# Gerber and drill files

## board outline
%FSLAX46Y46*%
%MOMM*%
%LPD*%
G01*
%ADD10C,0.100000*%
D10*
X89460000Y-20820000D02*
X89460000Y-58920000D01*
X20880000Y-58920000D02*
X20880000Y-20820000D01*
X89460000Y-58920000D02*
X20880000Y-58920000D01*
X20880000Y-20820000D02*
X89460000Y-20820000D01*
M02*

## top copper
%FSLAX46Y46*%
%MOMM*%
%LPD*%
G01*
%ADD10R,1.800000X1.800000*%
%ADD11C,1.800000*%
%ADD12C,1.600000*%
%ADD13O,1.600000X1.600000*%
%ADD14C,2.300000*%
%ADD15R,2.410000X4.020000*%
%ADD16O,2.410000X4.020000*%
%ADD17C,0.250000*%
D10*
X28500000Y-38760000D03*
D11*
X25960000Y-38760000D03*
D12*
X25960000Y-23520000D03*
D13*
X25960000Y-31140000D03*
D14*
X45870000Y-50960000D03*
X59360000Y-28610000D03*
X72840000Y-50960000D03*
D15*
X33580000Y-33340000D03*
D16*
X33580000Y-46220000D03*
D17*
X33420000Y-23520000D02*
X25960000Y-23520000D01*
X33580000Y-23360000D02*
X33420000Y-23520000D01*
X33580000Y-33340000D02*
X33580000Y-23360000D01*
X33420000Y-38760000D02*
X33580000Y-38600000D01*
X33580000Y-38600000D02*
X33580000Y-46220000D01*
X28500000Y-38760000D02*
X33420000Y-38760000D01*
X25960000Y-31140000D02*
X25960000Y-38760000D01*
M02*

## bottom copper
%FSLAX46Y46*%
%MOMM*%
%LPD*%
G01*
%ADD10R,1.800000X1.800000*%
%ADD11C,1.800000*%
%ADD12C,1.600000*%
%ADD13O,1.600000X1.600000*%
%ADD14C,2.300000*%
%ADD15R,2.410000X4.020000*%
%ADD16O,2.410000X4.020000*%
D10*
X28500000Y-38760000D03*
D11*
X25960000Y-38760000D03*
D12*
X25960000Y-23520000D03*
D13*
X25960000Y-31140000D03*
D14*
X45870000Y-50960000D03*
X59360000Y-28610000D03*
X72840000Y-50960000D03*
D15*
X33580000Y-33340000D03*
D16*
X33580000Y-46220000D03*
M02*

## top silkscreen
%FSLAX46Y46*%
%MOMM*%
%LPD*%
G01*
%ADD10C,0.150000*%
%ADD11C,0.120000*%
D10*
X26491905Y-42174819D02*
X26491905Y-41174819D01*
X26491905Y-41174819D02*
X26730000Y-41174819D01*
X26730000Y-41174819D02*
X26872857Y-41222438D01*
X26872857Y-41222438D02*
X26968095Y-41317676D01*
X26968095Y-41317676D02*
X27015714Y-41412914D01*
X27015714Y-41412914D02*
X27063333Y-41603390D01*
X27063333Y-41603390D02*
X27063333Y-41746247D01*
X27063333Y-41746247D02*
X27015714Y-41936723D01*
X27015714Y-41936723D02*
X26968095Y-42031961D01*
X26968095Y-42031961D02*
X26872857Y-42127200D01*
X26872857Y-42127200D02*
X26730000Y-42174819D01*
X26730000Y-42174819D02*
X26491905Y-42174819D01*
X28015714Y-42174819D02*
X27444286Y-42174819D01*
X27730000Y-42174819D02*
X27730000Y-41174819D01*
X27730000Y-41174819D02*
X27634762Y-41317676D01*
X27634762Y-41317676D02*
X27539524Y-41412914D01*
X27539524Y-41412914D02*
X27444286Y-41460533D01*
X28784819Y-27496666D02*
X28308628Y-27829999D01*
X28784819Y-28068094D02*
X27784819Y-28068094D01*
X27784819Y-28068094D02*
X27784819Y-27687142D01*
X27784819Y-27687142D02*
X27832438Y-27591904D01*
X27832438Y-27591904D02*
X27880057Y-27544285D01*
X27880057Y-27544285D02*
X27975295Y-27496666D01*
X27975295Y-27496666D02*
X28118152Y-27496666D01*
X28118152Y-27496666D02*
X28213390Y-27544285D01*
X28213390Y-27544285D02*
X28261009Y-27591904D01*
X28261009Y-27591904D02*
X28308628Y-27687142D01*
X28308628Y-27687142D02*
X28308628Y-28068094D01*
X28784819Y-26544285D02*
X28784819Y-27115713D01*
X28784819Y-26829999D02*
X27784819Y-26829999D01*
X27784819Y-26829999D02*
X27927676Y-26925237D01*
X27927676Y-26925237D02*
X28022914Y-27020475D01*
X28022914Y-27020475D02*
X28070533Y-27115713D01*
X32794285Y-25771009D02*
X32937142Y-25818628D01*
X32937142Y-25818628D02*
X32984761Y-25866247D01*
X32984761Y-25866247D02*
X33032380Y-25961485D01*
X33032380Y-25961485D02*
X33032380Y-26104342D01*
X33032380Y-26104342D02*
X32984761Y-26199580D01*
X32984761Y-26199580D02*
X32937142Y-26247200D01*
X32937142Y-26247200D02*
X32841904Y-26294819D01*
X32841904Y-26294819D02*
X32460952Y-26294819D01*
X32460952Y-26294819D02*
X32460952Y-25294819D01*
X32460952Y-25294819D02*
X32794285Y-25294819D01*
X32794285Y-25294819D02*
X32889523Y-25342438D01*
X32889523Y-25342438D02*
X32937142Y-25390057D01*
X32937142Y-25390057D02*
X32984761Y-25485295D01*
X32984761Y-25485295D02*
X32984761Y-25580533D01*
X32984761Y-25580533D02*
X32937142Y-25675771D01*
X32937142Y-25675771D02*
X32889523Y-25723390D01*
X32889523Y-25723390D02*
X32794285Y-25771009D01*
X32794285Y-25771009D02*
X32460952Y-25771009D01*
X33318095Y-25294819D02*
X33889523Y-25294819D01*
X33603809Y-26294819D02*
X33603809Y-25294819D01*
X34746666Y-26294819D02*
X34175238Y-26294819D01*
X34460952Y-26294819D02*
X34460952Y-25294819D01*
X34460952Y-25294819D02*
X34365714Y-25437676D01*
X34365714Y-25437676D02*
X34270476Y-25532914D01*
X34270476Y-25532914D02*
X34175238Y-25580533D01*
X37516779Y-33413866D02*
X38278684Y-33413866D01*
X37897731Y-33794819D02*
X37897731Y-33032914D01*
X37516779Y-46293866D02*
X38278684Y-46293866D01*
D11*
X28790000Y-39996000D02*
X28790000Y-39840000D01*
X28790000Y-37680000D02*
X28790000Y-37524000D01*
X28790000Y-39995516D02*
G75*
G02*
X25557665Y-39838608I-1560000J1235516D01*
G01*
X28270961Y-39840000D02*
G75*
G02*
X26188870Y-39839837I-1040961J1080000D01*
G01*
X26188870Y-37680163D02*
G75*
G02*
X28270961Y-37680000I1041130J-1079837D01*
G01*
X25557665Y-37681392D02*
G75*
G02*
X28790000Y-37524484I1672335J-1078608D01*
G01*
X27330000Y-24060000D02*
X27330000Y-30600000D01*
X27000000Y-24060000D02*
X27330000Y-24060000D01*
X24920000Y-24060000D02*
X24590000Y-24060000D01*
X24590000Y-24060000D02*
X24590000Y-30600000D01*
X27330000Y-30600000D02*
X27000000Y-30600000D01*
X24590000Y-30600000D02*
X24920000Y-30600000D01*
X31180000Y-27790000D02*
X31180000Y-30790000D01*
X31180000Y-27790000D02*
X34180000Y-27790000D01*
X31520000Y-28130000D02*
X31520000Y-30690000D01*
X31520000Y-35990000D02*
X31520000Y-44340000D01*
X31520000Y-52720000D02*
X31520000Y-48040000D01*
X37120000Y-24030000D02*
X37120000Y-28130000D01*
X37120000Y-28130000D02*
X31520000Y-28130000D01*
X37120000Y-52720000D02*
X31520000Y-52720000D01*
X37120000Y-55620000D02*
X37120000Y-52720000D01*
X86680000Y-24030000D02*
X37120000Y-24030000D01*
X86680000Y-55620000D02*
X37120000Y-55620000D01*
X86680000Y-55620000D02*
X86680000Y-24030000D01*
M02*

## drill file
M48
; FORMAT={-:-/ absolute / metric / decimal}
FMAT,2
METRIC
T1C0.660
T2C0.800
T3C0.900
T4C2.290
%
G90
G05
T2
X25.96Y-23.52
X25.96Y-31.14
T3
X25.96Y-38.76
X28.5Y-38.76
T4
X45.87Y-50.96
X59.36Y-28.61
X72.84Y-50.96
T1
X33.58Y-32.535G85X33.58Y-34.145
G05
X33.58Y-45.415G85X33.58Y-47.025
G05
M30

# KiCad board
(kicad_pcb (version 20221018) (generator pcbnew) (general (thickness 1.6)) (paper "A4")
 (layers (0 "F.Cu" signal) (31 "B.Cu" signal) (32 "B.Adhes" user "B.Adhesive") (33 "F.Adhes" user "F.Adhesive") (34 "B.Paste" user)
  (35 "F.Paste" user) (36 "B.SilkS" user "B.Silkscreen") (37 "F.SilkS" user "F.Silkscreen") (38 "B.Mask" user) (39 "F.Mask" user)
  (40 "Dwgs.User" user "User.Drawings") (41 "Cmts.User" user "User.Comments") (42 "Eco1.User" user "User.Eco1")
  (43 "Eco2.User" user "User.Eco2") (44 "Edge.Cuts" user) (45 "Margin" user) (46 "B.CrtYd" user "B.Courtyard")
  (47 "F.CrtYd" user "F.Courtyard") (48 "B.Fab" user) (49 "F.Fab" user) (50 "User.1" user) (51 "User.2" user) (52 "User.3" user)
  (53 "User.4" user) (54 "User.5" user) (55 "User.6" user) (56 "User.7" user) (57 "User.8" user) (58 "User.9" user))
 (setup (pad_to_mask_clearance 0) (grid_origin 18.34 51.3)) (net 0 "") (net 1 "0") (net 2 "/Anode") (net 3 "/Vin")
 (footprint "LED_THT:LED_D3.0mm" (layer "F.Cu") (at 28.5 38.76 180)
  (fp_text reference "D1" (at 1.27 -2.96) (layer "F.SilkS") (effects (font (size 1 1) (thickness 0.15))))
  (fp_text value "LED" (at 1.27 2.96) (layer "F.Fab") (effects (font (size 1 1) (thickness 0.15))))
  (fp_line (start -0.29 -1.236) (end -0.29 -1.08) (stroke (width 0.12) (type solid)) (layer "F.SilkS"))
  (fp_line (start -0.29 1.08) (end -0.29 1.236) (stroke (width 0.12) (type solid)) (layer "F.SilkS"))
  (fp_arc (start -0.29 -1.235516) (mid 1.366487 -1.987659) (end 2.942335 -1.078608) (stroke (width 0.12) (type solid)) (layer "F.SilkS"))
  (fp_arc (start 0.229039 -1.08) (mid 1.270117 -1.5) (end 2.31113 -1.079837) (stroke (width 0.12) (type solid)) (layer "F.SilkS"))
  (fp_arc (start 2.31113 1.079837) (mid 1.270117 1.5) (end 0.229039 1.08) (stroke (width 0.12) (type solid)) (layer "F.SilkS"))
  (fp_arc (start 2.942335 1.078608) (mid 1.366487 1.987659) (end -0.29 1.235516) (stroke (width 0.12) (type solid)) (layer "F.SilkS"))
  (pad "1" thru_hole rect (at 0 0 180) (size 1.8 1.8) (drill 0.9) (layers "*.Cu" "*.Mask") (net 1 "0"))
  (pad "2" thru_hole circle (at 2.54 0 180) (size 1.8 1.8) (drill 0.9) (layers "*.Cu" "*.Mask") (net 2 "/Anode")))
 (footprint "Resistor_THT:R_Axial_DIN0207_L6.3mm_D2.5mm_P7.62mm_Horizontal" (layer "F.Cu") (at 25.96 23.52 -90)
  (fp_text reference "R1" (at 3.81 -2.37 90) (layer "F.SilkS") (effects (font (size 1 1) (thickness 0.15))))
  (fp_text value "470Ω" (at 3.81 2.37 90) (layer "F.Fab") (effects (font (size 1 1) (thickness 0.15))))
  (fp_line (start 0.54 -1.37) (end 7.08 -1.37) (stroke (width 0.12) (type solid)) (layer "F.SilkS"))
  (fp_line (start 0.54 -1.04) (end 0.54 -1.37) (stroke (width 0.12) (type solid)) (layer "F.SilkS"))
  (fp_line (start 0.54 1.04) (end 0.54 1.37) (stroke (width 0.12) (type solid)) (layer "F.SilkS"))
  (fp_line (start 0.54 1.37) (end 7.08 1.37) (stroke (width 0.12) (type solid)) (layer "F.SilkS"))
  (fp_line (start 7.08 -1.37) (end 7.08 -1.04) (stroke (width 0.12) (type solid)) (layer "F.SilkS"))
  (fp_line (start 7.08 1.37) (end 7.08 1.04) (stroke (width 0.12) (type solid)) (layer "F.SilkS"))
  (pad "1" thru_hole circle (at 0 0 270) (size 1.6 1.6) (drill 0.8) (layers "*.Cu" "*.Mask") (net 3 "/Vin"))
  (pad "2" thru_hole oval (at 7.62 0 270) (size 1.6 1.6) (drill 0.8) (layers "*.Cu" "*.Mask") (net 2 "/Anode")))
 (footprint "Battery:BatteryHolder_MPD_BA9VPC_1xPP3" (layer "F.Cu") (at 33.58 33.34)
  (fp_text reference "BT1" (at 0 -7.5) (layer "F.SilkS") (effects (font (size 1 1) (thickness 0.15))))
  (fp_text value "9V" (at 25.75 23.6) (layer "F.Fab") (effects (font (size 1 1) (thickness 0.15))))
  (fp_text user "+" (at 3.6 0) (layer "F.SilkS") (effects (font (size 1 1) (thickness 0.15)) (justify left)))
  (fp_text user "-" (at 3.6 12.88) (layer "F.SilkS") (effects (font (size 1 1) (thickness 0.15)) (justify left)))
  (fp_line (start -2.4 -5.55) (end -2.4 -2.55) (stroke (width 0.12) (type solid)) (layer "F.SilkS"))
  (fp_line (start -2.4 -5.55) (end 0.6 -5.55) (stroke (width 0.12) (type solid)) (layer "F.SilkS"))
  (fp_line (start -2.06 -5.21) (end -2.06 -2.65) (stroke (width 0.12) (type solid)) (layer "F.SilkS"))
  (fp_line (start -2.06 2.65) (end -2.06 11) (stroke (width 0.12) (type solid)) (layer "F.SilkS"))
  (fp_line (start -2.06 19.38) (end -2.06 14.7) (stroke (width 0.12) (type solid)) (layer "F.SilkS"))
  (fp_line (start 3.54 -9.31) (end 3.54 -5.21) (stroke (width 0.12) (type solid)) (layer "F.SilkS"))
  (fp_line (start 3.54 -5.21) (end -2.06 -5.21) (stroke (width 0.12) (type solid)) (layer "F.SilkS"))
  (fp_line (start 3.54 19.38) (end -2.06 19.38) (stroke (width 0.12) (type solid)) (layer "F.SilkS"))
  (fp_line (start 3.54 22.28) (end 3.54 19.38) (stroke (width 0.12) (type solid)) (layer "F.SilkS"))
  (fp_line (start 53.1 -9.31) (end 3.54 -9.31) (stroke (width 0.12) (type solid)) (layer "F.SilkS"))
  (fp_line (start 53.1 22.28) (end 3.54 22.28) (stroke (width 0.12) (type solid)) (layer "F.SilkS"))
  (fp_line (start 53.1 22.28) (end 53.1 -9.31) (stroke (width 0.12) (type solid)) (layer "F.SilkS"))
  (pad "" np_thru_hole circle (at 12.29 17.62) (size 2.3 2.3) (drill 2.29) (layers "*.Cu" "*.Mask"))
  (pad "" np_thru_hole circle (at 25.78 -4.73) (size 2.3 2.3) (drill 2.29) (layers "*.Cu" "*.Mask"))
  (pad "" np_thru_hole circle (at 39.26 17.62) (size 2.3 2.3) (drill 2.29) (layers "*.Cu" "*.Mask"))
  (pad "1" thru_hole rect (at 0 0) (size 2.41 4.02) (drill oval 0.66 2.27) (layers "*.Cu" "*.Mask") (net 3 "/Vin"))
  (pad "2" thru_hole oval (at 0 12.88) (size 2.41 4.02) (drill oval 0.66 2.27) (layers "*.Cu" "*.Mask") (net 1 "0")))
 (gr_line (start 89.46 20.82) (end 89.46 58.92) (stroke (width 0.1) (type default)) (layer "Edge.Cuts"))
 (gr_line (start 20.88 58.92) (end 20.88 20.82) (stroke (width 0.1) (type default)) (layer "Edge.Cuts"))
 (gr_line (start 89.46 58.92) (end 20.88 58.92) (stroke (width 0.1) (type default)) (layer "Edge.Cuts"))
 (gr_line (start 20.88 20.82) (end 89.46 20.82) (stroke (width 0.1) (type default)) (layer "Edge.Cuts"))
 (segment (start 33.42 23.52) (end 25.96 23.52) (width 0.25) (layer "F.Cu") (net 3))
 (segment (start 33.58 23.36) (end 33.42 23.52) (width 0.25) (layer "F.Cu") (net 3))
 (segment (start 33.58 33.34) (end 33.58 23.36) (width 0.25) (layer "F.Cu") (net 3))
 (segment (start 33.42 38.76) (end 33.58 38.6) (width 0.25) (layer "F.Cu") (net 1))
 (segment (start 33.58 38.6) (end 33.58 46.22) (width 0.25) (layer "F.Cu") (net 1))
 (segment (start 28.5 38.76) (end 33.42 38.76) (width 0.25) (layer "F.Cu") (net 1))
 (segment (start 25.96 31.14) (end 25.96 38.76) (width 0.25) (layer "F.Cu") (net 2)))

